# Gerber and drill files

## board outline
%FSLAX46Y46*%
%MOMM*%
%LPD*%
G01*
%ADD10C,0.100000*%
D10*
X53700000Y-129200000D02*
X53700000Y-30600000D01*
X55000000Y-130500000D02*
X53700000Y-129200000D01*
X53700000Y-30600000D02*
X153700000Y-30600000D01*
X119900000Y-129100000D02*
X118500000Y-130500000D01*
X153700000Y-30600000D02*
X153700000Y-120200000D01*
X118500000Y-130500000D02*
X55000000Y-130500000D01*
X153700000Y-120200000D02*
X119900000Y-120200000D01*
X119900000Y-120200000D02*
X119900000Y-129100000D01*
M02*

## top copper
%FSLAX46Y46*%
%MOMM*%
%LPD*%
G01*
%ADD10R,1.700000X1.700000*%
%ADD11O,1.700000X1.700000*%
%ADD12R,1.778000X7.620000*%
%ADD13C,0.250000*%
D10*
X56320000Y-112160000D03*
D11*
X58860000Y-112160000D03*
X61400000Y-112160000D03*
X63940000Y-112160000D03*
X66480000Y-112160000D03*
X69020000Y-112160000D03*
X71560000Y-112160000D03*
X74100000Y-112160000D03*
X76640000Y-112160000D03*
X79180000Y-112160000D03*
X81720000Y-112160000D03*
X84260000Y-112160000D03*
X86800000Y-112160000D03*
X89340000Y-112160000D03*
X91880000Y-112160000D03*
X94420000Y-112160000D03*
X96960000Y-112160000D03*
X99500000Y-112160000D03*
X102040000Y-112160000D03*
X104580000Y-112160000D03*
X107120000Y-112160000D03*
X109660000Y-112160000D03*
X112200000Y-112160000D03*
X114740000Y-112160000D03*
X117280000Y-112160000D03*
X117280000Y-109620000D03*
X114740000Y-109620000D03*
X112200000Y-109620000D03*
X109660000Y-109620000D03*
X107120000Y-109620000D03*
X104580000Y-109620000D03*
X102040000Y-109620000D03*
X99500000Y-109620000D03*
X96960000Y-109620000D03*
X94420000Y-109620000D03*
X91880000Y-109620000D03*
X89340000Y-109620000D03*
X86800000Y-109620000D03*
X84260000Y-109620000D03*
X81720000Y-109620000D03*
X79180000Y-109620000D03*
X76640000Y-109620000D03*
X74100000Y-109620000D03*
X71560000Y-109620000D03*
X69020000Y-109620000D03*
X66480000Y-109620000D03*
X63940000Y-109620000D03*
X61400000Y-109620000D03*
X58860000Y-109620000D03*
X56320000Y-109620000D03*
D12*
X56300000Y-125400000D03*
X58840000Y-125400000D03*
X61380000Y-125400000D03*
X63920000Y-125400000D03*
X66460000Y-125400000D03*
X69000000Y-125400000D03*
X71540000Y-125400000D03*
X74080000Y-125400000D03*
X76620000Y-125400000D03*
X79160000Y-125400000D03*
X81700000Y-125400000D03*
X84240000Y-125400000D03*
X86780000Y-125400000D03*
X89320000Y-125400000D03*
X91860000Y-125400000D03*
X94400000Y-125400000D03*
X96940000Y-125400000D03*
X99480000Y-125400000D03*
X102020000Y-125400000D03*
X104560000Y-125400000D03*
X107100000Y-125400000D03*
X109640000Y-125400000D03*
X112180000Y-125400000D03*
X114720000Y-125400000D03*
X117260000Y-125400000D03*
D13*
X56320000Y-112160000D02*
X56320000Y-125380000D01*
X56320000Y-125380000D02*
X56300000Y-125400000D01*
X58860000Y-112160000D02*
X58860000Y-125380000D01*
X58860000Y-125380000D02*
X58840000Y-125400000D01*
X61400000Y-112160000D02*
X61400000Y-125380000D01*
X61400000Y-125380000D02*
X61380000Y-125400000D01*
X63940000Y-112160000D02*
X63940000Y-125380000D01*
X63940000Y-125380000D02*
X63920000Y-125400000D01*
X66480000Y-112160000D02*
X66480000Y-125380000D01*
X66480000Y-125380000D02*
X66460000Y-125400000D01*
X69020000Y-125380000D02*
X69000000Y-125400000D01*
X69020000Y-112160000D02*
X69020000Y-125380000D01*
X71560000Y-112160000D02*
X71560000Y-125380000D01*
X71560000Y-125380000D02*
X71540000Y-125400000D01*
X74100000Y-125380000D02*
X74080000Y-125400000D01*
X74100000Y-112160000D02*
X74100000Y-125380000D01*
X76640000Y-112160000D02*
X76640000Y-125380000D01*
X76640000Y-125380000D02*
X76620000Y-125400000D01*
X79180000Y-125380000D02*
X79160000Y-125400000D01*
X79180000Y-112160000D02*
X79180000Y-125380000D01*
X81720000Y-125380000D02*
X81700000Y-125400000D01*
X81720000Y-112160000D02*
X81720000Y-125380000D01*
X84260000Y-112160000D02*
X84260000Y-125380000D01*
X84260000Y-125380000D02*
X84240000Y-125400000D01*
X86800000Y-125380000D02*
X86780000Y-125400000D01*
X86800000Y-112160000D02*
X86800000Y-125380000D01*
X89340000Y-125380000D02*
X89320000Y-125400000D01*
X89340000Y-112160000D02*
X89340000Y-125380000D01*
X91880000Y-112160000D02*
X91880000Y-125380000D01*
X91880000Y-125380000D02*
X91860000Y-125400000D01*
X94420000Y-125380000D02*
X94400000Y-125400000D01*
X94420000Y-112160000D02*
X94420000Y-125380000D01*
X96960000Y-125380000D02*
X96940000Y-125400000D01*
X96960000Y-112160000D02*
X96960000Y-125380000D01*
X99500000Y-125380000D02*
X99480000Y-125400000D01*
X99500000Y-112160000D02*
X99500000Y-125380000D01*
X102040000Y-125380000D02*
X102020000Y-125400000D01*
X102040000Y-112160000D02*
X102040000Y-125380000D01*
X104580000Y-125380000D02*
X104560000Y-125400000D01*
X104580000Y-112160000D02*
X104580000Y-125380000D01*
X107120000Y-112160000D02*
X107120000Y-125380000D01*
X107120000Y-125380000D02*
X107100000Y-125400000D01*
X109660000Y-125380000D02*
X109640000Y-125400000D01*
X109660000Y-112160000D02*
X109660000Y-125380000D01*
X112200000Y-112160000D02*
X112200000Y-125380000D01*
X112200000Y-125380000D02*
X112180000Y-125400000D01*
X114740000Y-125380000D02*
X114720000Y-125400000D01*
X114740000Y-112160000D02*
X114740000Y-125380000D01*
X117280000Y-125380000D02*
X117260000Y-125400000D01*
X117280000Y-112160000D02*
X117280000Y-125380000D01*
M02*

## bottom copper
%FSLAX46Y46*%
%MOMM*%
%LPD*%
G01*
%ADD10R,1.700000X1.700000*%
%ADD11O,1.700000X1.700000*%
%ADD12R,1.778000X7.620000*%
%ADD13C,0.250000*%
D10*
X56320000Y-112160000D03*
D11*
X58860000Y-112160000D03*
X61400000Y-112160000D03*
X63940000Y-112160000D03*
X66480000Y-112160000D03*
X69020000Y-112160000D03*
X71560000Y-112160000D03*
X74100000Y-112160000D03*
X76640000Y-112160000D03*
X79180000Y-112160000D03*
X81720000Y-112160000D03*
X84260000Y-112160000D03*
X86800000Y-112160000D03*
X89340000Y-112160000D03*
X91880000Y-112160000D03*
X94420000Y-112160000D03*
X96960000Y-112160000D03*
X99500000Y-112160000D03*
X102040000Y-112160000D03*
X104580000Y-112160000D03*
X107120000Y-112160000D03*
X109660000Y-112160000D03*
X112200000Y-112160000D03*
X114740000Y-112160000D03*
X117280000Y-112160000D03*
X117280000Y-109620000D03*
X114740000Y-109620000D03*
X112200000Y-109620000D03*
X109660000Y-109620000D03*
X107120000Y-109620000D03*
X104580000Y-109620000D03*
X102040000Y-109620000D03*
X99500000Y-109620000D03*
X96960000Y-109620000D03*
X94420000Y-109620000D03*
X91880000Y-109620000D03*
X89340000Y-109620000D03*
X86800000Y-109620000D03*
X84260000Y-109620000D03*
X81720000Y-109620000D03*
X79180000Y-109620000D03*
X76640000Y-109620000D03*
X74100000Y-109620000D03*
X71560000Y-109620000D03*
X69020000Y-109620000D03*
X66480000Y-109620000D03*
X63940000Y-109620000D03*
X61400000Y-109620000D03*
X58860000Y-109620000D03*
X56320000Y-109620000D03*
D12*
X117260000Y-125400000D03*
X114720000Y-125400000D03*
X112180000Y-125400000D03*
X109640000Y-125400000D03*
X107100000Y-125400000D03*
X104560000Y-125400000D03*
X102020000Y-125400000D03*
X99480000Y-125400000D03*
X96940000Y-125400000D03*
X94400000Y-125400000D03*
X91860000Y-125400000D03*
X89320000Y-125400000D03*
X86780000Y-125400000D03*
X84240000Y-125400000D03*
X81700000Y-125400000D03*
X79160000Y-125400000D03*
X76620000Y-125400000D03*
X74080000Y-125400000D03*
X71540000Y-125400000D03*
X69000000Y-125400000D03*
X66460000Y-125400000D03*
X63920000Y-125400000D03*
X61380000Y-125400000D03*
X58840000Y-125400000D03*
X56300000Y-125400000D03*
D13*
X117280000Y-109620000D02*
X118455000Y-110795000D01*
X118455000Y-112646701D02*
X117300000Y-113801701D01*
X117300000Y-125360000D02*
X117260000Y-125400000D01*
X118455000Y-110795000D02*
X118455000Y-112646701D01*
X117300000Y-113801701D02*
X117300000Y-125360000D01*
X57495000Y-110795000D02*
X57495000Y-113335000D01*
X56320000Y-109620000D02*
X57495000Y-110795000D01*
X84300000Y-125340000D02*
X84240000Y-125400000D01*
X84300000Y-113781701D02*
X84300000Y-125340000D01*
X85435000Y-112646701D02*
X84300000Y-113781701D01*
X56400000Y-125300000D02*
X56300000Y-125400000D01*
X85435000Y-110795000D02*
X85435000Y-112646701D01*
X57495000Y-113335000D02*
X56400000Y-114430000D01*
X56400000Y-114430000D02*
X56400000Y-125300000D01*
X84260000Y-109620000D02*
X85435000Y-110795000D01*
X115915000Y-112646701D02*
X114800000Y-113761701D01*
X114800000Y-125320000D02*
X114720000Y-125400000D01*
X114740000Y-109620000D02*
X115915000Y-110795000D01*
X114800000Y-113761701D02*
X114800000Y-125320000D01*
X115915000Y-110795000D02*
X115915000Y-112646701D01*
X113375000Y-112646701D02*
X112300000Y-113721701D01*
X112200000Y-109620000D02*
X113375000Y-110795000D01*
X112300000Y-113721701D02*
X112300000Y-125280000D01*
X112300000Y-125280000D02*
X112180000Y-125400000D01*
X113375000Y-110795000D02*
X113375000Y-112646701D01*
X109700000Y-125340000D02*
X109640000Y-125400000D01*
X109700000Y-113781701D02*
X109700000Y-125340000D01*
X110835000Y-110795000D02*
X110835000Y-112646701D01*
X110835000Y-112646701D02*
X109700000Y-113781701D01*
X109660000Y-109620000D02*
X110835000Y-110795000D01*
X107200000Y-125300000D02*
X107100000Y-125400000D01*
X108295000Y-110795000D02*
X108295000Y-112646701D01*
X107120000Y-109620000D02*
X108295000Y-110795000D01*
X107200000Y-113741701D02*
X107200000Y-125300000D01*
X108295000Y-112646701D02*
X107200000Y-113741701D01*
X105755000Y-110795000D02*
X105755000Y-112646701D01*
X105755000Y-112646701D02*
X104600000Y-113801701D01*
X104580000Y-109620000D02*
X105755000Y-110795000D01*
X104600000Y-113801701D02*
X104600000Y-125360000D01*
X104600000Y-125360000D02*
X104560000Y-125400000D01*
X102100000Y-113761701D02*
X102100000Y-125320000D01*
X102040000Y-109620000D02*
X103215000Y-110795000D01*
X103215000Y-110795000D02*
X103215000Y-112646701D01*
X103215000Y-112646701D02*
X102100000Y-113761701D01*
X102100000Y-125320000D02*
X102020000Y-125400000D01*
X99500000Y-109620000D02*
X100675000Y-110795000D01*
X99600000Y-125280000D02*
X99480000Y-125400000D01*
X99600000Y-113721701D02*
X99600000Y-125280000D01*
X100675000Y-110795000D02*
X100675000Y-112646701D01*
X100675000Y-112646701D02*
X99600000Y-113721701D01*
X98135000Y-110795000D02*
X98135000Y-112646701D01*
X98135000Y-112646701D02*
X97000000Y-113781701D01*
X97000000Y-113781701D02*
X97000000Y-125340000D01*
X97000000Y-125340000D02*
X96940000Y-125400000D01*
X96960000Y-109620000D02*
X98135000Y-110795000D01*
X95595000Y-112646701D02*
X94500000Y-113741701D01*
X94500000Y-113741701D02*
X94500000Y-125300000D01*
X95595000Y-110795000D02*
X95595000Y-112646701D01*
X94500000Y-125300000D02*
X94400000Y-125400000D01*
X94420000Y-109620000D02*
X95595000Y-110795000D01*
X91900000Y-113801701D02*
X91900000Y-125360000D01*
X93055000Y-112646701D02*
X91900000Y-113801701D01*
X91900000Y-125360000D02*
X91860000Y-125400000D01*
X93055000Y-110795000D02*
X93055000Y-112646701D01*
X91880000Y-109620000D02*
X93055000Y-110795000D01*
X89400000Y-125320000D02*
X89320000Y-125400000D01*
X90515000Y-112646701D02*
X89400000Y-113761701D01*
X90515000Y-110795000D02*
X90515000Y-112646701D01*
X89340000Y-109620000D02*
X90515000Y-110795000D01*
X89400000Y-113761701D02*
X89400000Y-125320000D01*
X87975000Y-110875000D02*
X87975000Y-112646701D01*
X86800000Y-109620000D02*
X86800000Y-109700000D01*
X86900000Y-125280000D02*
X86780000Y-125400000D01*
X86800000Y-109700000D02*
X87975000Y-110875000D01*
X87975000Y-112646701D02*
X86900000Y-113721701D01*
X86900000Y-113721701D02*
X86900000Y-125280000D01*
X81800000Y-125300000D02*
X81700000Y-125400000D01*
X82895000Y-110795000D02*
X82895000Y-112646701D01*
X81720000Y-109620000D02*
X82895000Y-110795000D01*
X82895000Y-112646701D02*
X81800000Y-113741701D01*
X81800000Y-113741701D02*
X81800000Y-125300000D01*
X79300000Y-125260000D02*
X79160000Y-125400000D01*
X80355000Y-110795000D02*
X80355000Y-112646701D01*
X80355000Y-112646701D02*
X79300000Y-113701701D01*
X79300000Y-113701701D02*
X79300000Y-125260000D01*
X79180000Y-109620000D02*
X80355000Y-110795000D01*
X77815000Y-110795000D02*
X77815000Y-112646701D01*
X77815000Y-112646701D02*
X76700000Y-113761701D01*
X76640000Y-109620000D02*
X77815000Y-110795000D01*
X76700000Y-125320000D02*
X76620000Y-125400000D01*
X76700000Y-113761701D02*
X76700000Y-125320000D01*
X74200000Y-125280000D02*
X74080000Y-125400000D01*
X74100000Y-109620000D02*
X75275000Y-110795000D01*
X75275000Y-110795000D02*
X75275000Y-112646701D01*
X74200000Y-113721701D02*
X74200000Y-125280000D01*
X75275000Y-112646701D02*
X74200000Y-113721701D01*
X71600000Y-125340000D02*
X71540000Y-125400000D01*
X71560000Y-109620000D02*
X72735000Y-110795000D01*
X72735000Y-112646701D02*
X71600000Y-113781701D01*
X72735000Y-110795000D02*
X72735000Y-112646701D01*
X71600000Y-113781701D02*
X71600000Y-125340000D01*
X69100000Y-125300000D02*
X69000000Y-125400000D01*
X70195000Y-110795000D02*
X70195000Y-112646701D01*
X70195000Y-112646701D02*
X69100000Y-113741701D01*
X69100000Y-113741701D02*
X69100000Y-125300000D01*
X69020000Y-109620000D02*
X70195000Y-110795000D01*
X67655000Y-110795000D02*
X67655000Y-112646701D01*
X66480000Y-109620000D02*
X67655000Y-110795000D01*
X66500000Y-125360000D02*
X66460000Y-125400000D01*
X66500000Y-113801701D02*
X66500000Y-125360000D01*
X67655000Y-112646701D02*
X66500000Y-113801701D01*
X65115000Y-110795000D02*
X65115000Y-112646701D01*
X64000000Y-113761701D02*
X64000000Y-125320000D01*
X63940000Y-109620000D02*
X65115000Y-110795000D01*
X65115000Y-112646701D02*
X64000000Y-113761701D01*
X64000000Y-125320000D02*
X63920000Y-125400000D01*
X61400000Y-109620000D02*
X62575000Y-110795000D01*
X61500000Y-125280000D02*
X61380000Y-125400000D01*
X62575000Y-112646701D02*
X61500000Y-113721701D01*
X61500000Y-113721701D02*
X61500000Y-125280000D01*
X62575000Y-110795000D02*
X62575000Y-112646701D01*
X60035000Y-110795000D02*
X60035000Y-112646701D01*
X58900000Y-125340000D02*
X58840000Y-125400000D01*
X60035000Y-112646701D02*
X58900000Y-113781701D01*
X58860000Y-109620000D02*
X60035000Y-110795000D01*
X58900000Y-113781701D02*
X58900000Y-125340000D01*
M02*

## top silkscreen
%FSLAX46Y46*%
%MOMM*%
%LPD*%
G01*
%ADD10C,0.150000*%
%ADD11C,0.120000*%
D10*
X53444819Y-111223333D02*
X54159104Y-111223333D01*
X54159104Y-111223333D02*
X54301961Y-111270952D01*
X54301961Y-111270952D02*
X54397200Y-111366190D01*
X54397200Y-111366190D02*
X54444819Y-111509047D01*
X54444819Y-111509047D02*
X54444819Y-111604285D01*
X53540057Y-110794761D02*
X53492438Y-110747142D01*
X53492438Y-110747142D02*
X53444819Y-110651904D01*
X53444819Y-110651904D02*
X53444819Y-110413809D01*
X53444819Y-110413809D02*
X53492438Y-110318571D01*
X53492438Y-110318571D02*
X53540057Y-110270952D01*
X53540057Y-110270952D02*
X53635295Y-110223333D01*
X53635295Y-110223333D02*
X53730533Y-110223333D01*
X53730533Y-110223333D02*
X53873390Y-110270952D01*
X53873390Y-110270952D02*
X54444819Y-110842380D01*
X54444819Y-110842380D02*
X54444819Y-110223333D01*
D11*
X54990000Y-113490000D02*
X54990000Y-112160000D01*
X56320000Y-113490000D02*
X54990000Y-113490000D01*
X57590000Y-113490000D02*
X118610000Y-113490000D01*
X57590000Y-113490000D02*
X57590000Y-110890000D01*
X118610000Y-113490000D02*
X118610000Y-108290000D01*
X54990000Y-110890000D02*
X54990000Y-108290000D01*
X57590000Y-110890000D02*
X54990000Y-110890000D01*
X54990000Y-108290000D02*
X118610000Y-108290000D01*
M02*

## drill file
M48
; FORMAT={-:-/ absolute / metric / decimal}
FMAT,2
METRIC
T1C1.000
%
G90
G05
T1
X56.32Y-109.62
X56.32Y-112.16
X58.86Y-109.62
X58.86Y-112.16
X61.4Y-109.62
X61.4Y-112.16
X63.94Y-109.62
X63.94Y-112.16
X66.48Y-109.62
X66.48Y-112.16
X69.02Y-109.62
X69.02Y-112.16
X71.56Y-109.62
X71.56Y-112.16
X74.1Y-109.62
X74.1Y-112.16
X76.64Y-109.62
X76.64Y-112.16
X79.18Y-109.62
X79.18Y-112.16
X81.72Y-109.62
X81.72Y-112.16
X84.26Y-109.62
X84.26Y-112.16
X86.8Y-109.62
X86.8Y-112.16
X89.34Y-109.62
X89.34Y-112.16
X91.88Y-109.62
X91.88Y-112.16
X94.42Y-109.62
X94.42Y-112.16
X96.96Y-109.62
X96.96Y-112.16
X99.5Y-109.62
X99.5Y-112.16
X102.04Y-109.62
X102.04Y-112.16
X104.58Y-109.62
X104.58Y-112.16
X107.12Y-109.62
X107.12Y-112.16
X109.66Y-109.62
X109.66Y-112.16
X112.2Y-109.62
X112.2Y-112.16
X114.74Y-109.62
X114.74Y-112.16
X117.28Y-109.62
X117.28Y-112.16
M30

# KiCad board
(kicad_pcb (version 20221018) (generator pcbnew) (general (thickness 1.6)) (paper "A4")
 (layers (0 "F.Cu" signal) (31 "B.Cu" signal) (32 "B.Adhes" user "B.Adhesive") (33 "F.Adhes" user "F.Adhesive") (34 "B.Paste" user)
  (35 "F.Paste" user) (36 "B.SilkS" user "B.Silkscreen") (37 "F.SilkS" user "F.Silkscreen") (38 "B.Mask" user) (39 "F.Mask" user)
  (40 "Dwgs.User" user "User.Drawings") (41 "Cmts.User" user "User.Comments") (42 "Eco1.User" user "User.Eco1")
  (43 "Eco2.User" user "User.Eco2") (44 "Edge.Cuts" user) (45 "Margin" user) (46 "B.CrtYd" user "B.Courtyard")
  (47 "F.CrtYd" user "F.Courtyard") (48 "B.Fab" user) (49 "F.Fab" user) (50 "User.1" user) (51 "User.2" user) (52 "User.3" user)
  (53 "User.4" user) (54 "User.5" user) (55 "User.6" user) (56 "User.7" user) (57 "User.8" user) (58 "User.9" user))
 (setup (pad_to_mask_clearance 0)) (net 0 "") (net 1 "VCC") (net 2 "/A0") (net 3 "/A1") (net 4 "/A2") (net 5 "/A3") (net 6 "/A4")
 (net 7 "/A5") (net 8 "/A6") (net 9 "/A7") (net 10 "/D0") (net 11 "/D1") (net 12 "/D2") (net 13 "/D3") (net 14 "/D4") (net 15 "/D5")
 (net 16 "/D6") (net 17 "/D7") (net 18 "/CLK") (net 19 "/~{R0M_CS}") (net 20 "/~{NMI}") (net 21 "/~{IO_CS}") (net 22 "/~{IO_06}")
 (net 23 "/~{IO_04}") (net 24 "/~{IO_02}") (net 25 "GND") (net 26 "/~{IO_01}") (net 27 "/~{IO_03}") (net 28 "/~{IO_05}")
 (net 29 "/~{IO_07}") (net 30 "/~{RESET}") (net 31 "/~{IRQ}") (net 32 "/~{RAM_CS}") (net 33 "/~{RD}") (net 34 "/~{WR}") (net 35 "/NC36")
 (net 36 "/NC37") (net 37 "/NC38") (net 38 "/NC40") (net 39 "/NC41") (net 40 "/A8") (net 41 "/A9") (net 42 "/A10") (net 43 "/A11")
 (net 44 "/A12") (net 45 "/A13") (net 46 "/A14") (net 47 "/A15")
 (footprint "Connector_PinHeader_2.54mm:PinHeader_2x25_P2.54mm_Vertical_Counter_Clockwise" (layer "F.Cu") (at 56.32 112.16 90)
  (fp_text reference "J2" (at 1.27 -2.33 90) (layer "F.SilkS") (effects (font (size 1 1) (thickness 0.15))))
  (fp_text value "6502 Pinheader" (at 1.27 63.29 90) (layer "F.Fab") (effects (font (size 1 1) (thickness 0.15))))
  (fp_line (start -1.33 -1.33) (end 0 -1.33) (stroke (width 0.12) (type solid)) (layer "F.SilkS"))
  (fp_line (start -1.33 0) (end -1.33 -1.33) (stroke (width 0.12) (type solid)) (layer "F.SilkS"))
  (fp_line (start -1.33 1.27) (end -1.33 62.29) (stroke (width 0.12) (type solid)) (layer "F.SilkS"))
  (fp_line (start -1.33 1.27) (end 1.27 1.27) (stroke (width 0.12) (type solid)) (layer "F.SilkS"))
  (fp_line (start -1.33 62.29) (end 3.87 62.29) (stroke (width 0.12) (type solid)) (layer "F.SilkS"))
  (fp_line (start 1.27 -1.33) (end 3.87 -1.33) (stroke (width 0.12) (type solid)) (layer "F.SilkS"))
  (fp_line (start 1.27 1.27) (end 1.27 -1.33) (stroke (width 0.12) (type solid)) (layer "F.SilkS"))
  (fp_line (start 3.87 -1.33) (end 3.87 62.29) (stroke (width 0.12) (type solid)) (layer "F.SilkS"))
  (pad "1" thru_hole rect (at 0 0 90) (size 1.7 1.7) (drill 1) (layers "*.Cu" "*.Mask") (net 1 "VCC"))
  (pad "2" thru_hole oval (at 0 2.54 90) (size 1.7 1.7) (drill 1) (layers "*.Cu" "*.Mask") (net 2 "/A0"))
  (pad "3" thru_hole oval (at 0 5.08 90) (size 1.7 1.7) (drill 1) (layers "*.Cu" "*.Mask") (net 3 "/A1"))
  (pad "4" thru_hole oval (at 0 7.62 90) (size 1.7 1.7) (drill 1) (layers "*.Cu" "*.Mask") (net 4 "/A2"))
  (pad "5" thru_hole oval (at 0 10.16 90) (size 1.7 1.7) (drill 1) (layers "*.Cu" "*.Mask") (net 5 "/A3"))
  (pad "6" thru_hole oval (at 0 12.7 90) (size 1.7 1.7) (drill 1) (layers "*.Cu" "*.Mask") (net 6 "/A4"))
  (pad "7" thru_hole oval (at 0 15.24 90) (size 1.7 1.7) (drill 1) (layers "*.Cu" "*.Mask") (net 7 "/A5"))
  (pad "8" thru_hole oval (at 0 17.78 90) (size 1.7 1.7) (drill 1) (layers "*.Cu" "*.Mask") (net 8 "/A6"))
  (pad "9" thru_hole oval (at 0 20.32 90) (size 1.7 1.7) (drill 1) (layers "*.Cu" "*.Mask") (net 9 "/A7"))
  (pad "10" thru_hole oval (at 0 22.86 90) (size 1.7 1.7) (drill 1) (layers "*.Cu" "*.Mask") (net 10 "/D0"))
  (pad "11" thru_hole oval (at 0 25.4 90) (size 1.7 1.7) (drill 1) (layers "*.Cu" "*.Mask") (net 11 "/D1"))
  (pad "12" thru_hole oval (at 0 27.94 90) (size 1.7 1.7) (drill 1) (layers "*.Cu" "*.Mask") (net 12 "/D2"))
  (pad "13" thru_hole oval (at 0 30.48 90) (size 1.7 1.7) (drill 1) (layers "*.Cu" "*.Mask") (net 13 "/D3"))
  (pad "14" thru_hole oval (at 0 33.02 90) (size 1.7 1.7) (drill 1) (layers "*.Cu" "*.Mask") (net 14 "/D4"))
  (pad "15" thru_hole oval (at 0 35.56 90) (size 1.7 1.7) (drill 1) (layers "*.Cu" "*.Mask") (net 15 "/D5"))
  (pad "16" thru_hole oval (at 0 38.1 90) (size 1.7 1.7) (drill 1) (layers "*.Cu" "*.Mask") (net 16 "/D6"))
  (pad "17" thru_hole oval (at 0 40.64 90) (size 1.7 1.7) (drill 1) (layers "*.Cu" "*.Mask") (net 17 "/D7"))
  (pad "18" thru_hole oval (at 0 43.18 90) (size 1.7 1.7) (drill 1) (layers "*.Cu" "*.Mask") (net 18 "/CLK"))
  (pad "19" thru_hole oval (at 0 45.72 90) (size 1.7 1.7) (drill 1) (layers "*.Cu" "*.Mask") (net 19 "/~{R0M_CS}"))
  (pad "20" thru_hole oval (at 0 48.26 90) (size 1.7 1.7) (drill 1) (layers "*.Cu" "*.Mask") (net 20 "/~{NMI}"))
  (pad "21" thru_hole oval (at 0 50.8 90) (size 1.7 1.7) (drill 1) (layers "*.Cu" "*.Mask") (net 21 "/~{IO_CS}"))
  (pad "22" thru_hole oval (at 0 53.34 90) (size 1.7 1.7) (drill 1) (layers "*.Cu" "*.Mask") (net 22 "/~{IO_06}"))
  (pad "23" thru_hole oval (at 0 55.88 90) (size 1.7 1.7) (drill 1) (layers "*.Cu" "*.Mask") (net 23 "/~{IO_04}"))
  (pad "24" thru_hole oval (at 0 58.42 90) (size 1.7 1.7) (drill 1) (layers "*.Cu" "*.Mask") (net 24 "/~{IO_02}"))
  (pad "25" thru_hole oval (at 0 60.96 90) (size 1.7 1.7) (drill 1) (layers "*.Cu" "*.Mask") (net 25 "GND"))
  (pad "26" thru_hole oval (at 2.54 60.96 90) (size 1.7 1.7) (drill 1) (layers "*.Cu" "*.Mask") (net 1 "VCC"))
  (pad "27" thru_hole oval (at 2.54 58.42 90) (size 1.7 1.7) (drill 1) (layers "*.Cu" "*.Mask") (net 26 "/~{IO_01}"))
  (pad "28" thru_hole oval (at 2.54 55.88 90) (size 1.7 1.7) (drill 1) (layers "*.Cu" "*.Mask") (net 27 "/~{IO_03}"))
  (pad "29" thru_hole oval (at 2.54 53.34 90) (size 1.7 1.7) (drill 1) (layers "*.Cu" "*.Mask") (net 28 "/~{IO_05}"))
  (pad "30" thru_hole oval (at 2.54 50.8 90) (size 1.7 1.7) (drill 1) (layers "*.Cu" "*.Mask") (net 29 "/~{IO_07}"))
  (pad "31" thru_hole oval (at 2.54 48.26 90) (size 1.7 1.7) (drill 1) (layers "*.Cu" "*.Mask") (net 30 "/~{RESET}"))
  (pad "32" thru_hole oval (at 2.54 45.72 90) (size 1.7 1.7) (drill 1) (layers "*.Cu" "*.Mask") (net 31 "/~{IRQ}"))
  (pad "33" thru_hole oval (at 2.54 43.18 90) (size 1.7 1.7) (drill 1) (layers "*.Cu" "*.Mask") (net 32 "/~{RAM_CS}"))
  (pad "34" thru_hole oval (at 2.54 40.64 90) (size 1.7 1.7) (drill 1) (layers "*.Cu" "*.Mask") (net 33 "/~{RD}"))
  (pad "35" thru_hole oval (at 2.54 38.1 90) (size 1.7 1.7) (drill 1) (layers "*.Cu" "*.Mask") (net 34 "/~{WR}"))
  (pad "36" thru_hole oval (at 2.54 35.56 90) (size 1.7 1.7) (drill 1) (layers "*.Cu" "*.Mask") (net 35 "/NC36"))
  (pad "37" thru_hole oval (at 2.54 33.02 90) (size 1.7 1.7) (drill 1) (layers "*.Cu" "*.Mask") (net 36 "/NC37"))
  (pad "38" thru_hole oval (at 2.54 30.48 90) (size 1.7 1.7) (drill 1) (layers "*.Cu" "*.Mask") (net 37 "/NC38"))
  (pad "39" thru_hole oval (at 2.54 27.94 90) (size 1.7 1.7) (drill 1) (layers "*.Cu" "*.Mask") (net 25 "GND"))
  (pad "40" thru_hole oval (at 2.54 25.4 90) (size 1.7 1.7) (drill 1) (layers "*.Cu" "*.Mask") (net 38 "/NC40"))
  (pad "41" thru_hole oval (at 2.54 22.86 90) (size 1.7 1.7) (drill 1) (layers "*.Cu" "*.Mask") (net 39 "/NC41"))
  (pad "42" thru_hole oval (at 2.54 20.32 90) (size 1.7 1.7) (drill 1) (layers "*.Cu" "*.Mask") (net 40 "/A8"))
  (pad "43" thru_hole oval (at 2.54 17.78 90) (size 1.7 1.7) (drill 1) (layers "*.Cu" "*.Mask") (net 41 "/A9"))
  (pad "44" thru_hole oval (at 2.54 15.24 90) (size 1.7 1.7) (drill 1) (layers "*.Cu" "*.Mask") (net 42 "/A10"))
  (pad "45" thru_hole oval (at 2.54 12.7 90) (size 1.7 1.7) (drill 1) (layers "*.Cu" "*.Mask") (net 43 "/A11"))
  (pad "46" thru_hole oval (at 2.54 10.16 90) (size 1.7 1.7) (drill 1) (layers "*.Cu" "*.Mask") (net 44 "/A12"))
  (pad "47" thru_hole oval (at 2.54 7.62 90) (size 1.7 1.7) (drill 1) (layers "*.Cu" "*.Mask") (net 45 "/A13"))
  (pad "48" thru_hole oval (at 2.54 5.08 90) (size 1.7 1.7) (drill 1) (layers "*.Cu" "*.Mask") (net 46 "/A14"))
  (pad "49" thru_hole oval (at 2.54 2.54 90) (size 1.7 1.7) (drill 1) (layers "*.Cu" "*.Mask") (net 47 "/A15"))
  (pad "50" thru_hole oval (at 2.54 0 90) (size 1.7 1.7) (drill 1) (layers "*.Cu" "*.Mask") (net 25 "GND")))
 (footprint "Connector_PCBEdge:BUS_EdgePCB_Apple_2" (layer "F.Cu") (at 79.16 125.4)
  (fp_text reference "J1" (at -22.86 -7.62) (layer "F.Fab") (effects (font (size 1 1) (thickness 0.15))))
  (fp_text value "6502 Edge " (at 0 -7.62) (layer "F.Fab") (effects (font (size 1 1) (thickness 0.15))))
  (pad "1" connect rect (at -22.86 0 180) (size 1.778 7.62) (layers "F.Cu" "F.Mask") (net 1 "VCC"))
  (pad "2" connect rect (at -20.32 0 180) (size 1.778 7.62) (layers "F.Cu" "F.Mask") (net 2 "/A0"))
  (pad "3" connect rect (at -17.78 0 180) (size 1.778 7.62) (layers "F.Cu" "F.Mask") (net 3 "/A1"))
  (pad "4" connect rect (at -15.24 0 180) (size 1.778 7.62) (layers "F.Cu" "F.Mask") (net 4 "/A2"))
  (pad "5" connect rect (at -12.7 0 180) (size 1.778 7.62) (layers "F.Cu" "F.Mask") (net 5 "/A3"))
  (pad "6" connect rect (at -10.16 0 180) (size 1.778 7.62) (layers "F.Cu" "F.Mask") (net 6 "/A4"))
  (pad "7" connect rect (at -7.62 0 180) (size 1.778 7.62) (layers "F.Cu" "F.Mask") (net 7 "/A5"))
  (pad "8" connect rect (at -5.08 0 180) (size 1.778 7.62) (layers "F.Cu" "F.Mask") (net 8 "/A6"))
  (pad "9" connect rect (at -2.54 0 180) (size 1.778 7.62) (layers "F.Cu" "F.Mask") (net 9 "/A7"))
  (pad "10" connect rect (at 0 0 180) (size 1.778 7.62) (layers "F.Cu" "F.Mask") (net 10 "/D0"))
  (pad "11" connect rect (at 2.54 0 180) (size 1.778 7.62) (layers "F.Cu" "F.Mask") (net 11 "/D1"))
  (pad "12" connect rect (at 5.08 0 180) (size 1.778 7.62) (layers "F.Cu" "F.Mask") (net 12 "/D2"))
  (pad "13" connect rect (at 7.62 0 180) (size 1.778 7.62) (layers "F.Cu" "F.Mask") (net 13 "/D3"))
  (pad "14" connect rect (at 10.16 0 180) (size 1.778 7.62) (layers "F.Cu" "F.Mask") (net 14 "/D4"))
  (pad "15" connect rect (at 12.7 0 180) (size 1.778 7.62) (layers "F.Cu" "F.Mask") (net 15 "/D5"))
  (pad "16" connect rect (at 15.24 0 180) (size 1.778 7.62) (layers "F.Cu" "F.Mask") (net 16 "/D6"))
  (pad "17" connect rect (at 17.78 0 180) (size 1.778 7.62) (layers "F.Cu" "F.Mask") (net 17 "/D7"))
  (pad "18" connect rect (at 20.32 0 180) (size 1.778 7.62) (layers "F.Cu" "F.Mask") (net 18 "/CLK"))
  (pad "19" connect rect (at 22.86 0 180) (size 1.778 7.62) (layers "F.Cu" "F.Mask") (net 19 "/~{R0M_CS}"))
  (pad "20" connect rect (at 25.4 0 180) (size 1.778 7.62) (layers "F.Cu" "F.Mask") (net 20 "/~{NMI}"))
  (pad "21" connect rect (at 27.94 0 180) (size 1.778 7.62) (layers "F.Cu" "F.Mask") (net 21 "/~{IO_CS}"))
  (pad "22" connect rect (at 30.48 0 180) (size 1.778 7.62) (layers "F.Cu" "F.Mask") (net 22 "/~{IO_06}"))
  (pad "23" connect rect (at 33.02 0 180) (size 1.778 7.62) (layers "F.Cu" "F.Mask") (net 23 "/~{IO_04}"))
  (pad "24" connect rect (at 35.56 0 180) (size 1.778 7.62) (layers "F.Cu" "F.Mask") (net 24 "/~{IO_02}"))
  (pad "25" connect rect (at 38.1 0 180) (size 1.778 7.62) (layers "F.Cu" "F.Mask") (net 25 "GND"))
  (pad "26" connect rect (at 38.1 0 180) (size 1.778 7.62) (layers "B.Cu" "B.Mask") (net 1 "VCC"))
  (pad "27" connect rect (at 35.56 0 180) (size 1.778 7.62) (layers "B.Cu" "B.Mask") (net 26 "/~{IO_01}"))
  (pad "28" connect rect (at 33.02 0 180) (size 1.778 7.62) (layers "B.Cu" "B.Mask") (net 27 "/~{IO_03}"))
  (pad "29" connect rect (at 30.48 0 180) (size 1.778 7.62) (layers "B.Cu" "B.Mask") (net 28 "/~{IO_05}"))
  (pad "30" connect rect (at 27.94 0 180) (size 1.778 7.62) (layers "B.Cu" "B.Mask") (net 29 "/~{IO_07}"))
  (pad "31" connect rect (at 25.4 0 180) (size 1.778 7.62) (layers "B.Cu" "B.Mask") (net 30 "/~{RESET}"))
  (pad "32" connect rect (at 22.86 0 180) (size 1.778 7.62) (layers "B.Cu" "B.Mask") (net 31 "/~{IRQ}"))
  (pad "33" connect rect (at 20.32 0 180) (size 1.778 7.62) (layers "B.Cu" "B.Mask") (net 32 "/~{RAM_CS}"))
  (pad "34" connect rect (at 17.78 0 180) (size 1.778 7.62) (layers "B.Cu" "B.Mask") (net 33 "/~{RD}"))
  (pad "35" connect rect (at 15.24 0 180) (size 1.778 7.62) (layers "B.Cu" "B.Mask") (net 34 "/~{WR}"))
  (pad "36" connect rect (at 12.7 0 180) (size 1.778 7.62) (layers "B.Cu" "B.Mask") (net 35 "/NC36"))
  (pad "37" connect rect (at 10.16 0 180) (size 1.778 7.62) (layers "B.Cu" "B.Mask") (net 36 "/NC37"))
  (pad "38" connect rect (at 7.62 0 180) (size 1.778 7.62) (layers "B.Cu" "B.Mask") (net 37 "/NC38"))
  (pad "39" connect rect (at 5.08 0 180) (size 1.778 7.62) (layers "B.Cu" "B.Mask") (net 25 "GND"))
  (pad "40" connect rect (at 2.54 0 180) (size 1.778 7.62) (layers "B.Cu" "B.Mask") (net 38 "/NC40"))
  (pad "41" connect rect (at 0 0 180) (size 1.778 7.62) (layers "B.Cu" "B.Mask") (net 39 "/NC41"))
  (pad "42" connect rect (at -2.54 0 180) (size 1.778 7.62) (layers "B.Cu" "B.Mask") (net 40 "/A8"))
  (pad "43" connect rect (at -5.08 0 180) (size 1.778 7.62) (layers "B.Cu" "B.Mask") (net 41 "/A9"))
  (pad "44" connect rect (at -7.62 0 180) (size 1.778 7.62) (layers "B.Cu" "B.Mask") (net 42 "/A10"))
  (pad "45" connect rect (at -10.16 0 180) (size 1.778 7.62) (layers "B.Cu" "B.Mask") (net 43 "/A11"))
  (pad "46" connect rect (at -12.7 0 180) (size 1.778 7.62) (layers "B.Cu" "B.Mask") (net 44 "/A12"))
  (pad "47" connect rect (at -15.24 0 180) (size 1.778 7.62) (layers "B.Cu" "B.Mask") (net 45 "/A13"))
  (pad "48" connect rect (at -17.78 0 180) (size 1.778 7.62) (layers "B.Cu" "B.Mask") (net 46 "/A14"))
  (pad "49" connect rect (at -20.32 0 180) (size 1.778 7.62) (layers "B.Cu" "B.Mask") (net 47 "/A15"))
  (pad "50" connect rect (at -22.86 0 180) (size 1.778 7.62) (layers "B.Cu" "B.Mask") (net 25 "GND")))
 (gr_line (start 53.7 129.2) (end 53.7 30.6) (stroke (width 0.1) (type default)) (layer "Edge.Cuts"))
 (gr_line (start 55 130.5) (end 53.7 129.2) (stroke (width 0.1) (type default)) (layer "Edge.Cuts"))
 (gr_line (start 53.7 30.6) (end 153.7 30.6) (stroke (width 0.1) (type default)) (layer "Edge.Cuts"))
 (gr_line (start 119.9 129.1) (end 118.5 130.5) (stroke (width 0.1) (type default)) (layer "Edge.Cuts"))
 (gr_line (start 153.7 30.6) (end 153.7 120.2) (stroke (width 0.1) (type default)) (layer "Edge.Cuts"))
 (gr_line (start 118.5 130.5) (end 55 130.5) (stroke (width 0.1) (type default)) (layer "Edge.Cuts"))
 (gr_line (start 153.7 120.2) (end 119.9 120.2) (stroke (width 0.1) (type default)) (layer "Edge.Cuts"))
 (gr_line (start 119.9 120.2) (end 119.9 129.1) (stroke (width 0.1) (type default)) (layer "Edge.Cuts"))
 (segment (start 56.32 112.16) (end 56.32 125.38) (width 0.25) (layer "F.Cu") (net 1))
 (segment (start 56.32 125.38) (end 56.3 125.4) (width 0.25) (layer "F.Cu") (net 1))
 (segment (start 117.28 109.62) (end 118.455 110.795) (width 0.25) (layer "B.Cu") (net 1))
 (segment (start 118.455 112.646701) (end 117.3 113.801701) (width 0.25) (layer "B.Cu") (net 1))
 (segment (start 117.3 125.36) (end 117.26 125.4) (width 0.25) (layer "B.Cu") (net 1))
 (segment (start 118.455 110.795) (end 118.455 112.646701) (width 0.25) (layer "B.Cu") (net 1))
 (segment (start 117.3 113.801701) (end 117.3 125.36) (width 0.25) (layer "B.Cu") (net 1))
 (segment (start 58.86 112.16) (end 58.86 125.38) (width 0.25) (layer "F.Cu") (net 2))
 (segment (start 58.86 125.38) (end 58.84 125.4) (width 0.25) (layer "F.Cu") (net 2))
 (segment (start 61.4 112.16) (end 61.4 125.38) (width 0.25) (layer "F.Cu") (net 3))
 (segment (start 61.4 125.38) (end 61.38 125.4) (width 0.25) (layer "F.Cu") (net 3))
 (segment (start 63.94 112.16) (end 63.94 125.38) (width 0.25) (layer "F.Cu") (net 4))
 (segment (start 63.94 125.38) (end 63.92 125.4) (width 0.25) (layer "F.Cu") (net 4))
 (segment (start 66.48 112.16) (end 66.48 125.38) (width 0.25) (layer "F.Cu") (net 5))
 (segment (start 66.48 125.38) (end 66.46 125.4) (width 0.25) (layer "F.Cu") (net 5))
 (segment (start 69.02 125.38) (end 69 125.4) (width 0.25) (layer "F.Cu") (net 6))
 (segment (start 69.02 112.16) (end 69.02 125.38) (width 0.25) (layer "F.Cu") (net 6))
 (segment (start 71.56 112.16) (end 71.56 125.38) (width 0.25) (layer "F.Cu") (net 7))
 (segment (start 71.56 125.38) (end 71.54 125.4) (width 0.25) (layer "F.Cu") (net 7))
 (segment (start 74.1 125.38) (end 74.08 125.4) (width 0.25) (layer "F.Cu") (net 8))
 (segment (start 74.1 112.16) (end 74.1 125.38) (width 0.25) (layer "F.Cu") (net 8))
 (segment (start 76.64 112.16) (end 76.64 125.38) (width 0.25) (layer "F.Cu") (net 9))
 (segment (start 76.64 125.38) (end 76.62 125.4) (width 0.25) (layer "F.Cu") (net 9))
 (segment (start 79.18 125.38) (end 79.16 125.4) (width 0.25) (layer "F.Cu") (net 10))
 (segment (start 79.18 112.16) (end 79.18 125.38) (width 0.25) (layer "F.Cu") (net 10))
 (segment (start 81.72 125.38) (end 81.7 125.4) (width 0.25) (layer "F.Cu") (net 11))
 (segment (start 81.72 112.16) (end 81.72 125.38) (width 0.25) (layer "F.Cu") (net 11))
 (segment (start 84.26 112.16) (end 84.26 125.38) (width 0.25) (layer "F.Cu") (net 12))
 (segment (start 84.26 125.38) (end 84.24 125.4) (width 0.25) (layer "F.Cu") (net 12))
 (segment (start 86.8 125.38) (end 86.78 125.4) (width 0.25) (layer "F.Cu") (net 13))
 (segment (start 86.8 112.16) (end 86.8 125.38) (width 0.25) (layer "F.Cu") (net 13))
 (segment (start 89.34 125.38) (end 89.32 125.4) (width 0.25) (layer "F.Cu") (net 14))
 (segment (start 89.34 112.16) (end 89.34 125.38) (width 0.25) (layer "F.Cu") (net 14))
 (segment (start 91.88 112.16) (end 91.88 125.38) (width 0.25) (layer "F.Cu") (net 15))
 (segment (start 91.88 125.38) (end 91.86 125.4) (width 0.25) (layer "F.Cu") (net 15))
 (segment (start 94.42 125.38) (end 94.4 125.4) (width 0.25) (layer "F.Cu") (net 16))
 (segment (start 94.42 112.16) (end 94.42 125.38) (width 0.25) (layer "F.Cu") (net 16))
 (segment (start 96.96 125.38) (end 96.94 125.4) (width 0.25) (layer "F.Cu") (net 17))
 (segment (start 96.96 112.16) (end 96.96 125.38) (width 0.25) (layer "F.Cu") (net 17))
 (segment (start 99.5 125.38) (end 99.48 125.4) (width 0.25) (layer "F.Cu") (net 18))
 (segment (start 99.5 112.16) (end 99.5 125.38) (width 0.25) (layer "F.Cu") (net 18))
 (segment (start 102.04 125.38) (end 102.02 125.4) (width 0.25) (layer "F.Cu") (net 19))
 (segment (start 102.04 112.16) (end 102.04 125.38) (width 0.25) (layer "F.Cu") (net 19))
 (segment (start 104.58 125.38) (end 104.56 125.4) (width 0.25) (layer "F.Cu") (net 20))
 (segment (start 104.58 112.16) (end 104.58 125.38) (width 0.25) (layer "F.Cu") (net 20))
 (segment (start 107.12 112.16) (end 107.12 125.38) (width 0.25) (layer "F.Cu") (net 21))
 (segment (start 107.12 125.38) (end 107.1 125.4) (width 0.25) (layer "F.Cu") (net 21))
 (segment (start 109.66 125.38) (end 109.64 125.4) (width 0.25) (layer "F.Cu") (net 22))
 (segment (start 109.66 112.16) (end 109.66 125.38) (width 0.25) (layer "F.Cu") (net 22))
 (segment (start 112.2 112.16) (end 112.2 125.38) (width 0.25) (layer "F.Cu") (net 23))
 (segment (start 112.2 125.38) (end 112.18 125.4) (width 0.25) (layer "F.Cu") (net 23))
 (segment (start 114.74 125.38) (end 114.72 125.4) (width 0.25) (layer "F.Cu") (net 24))
 (segment (start 114.74 112.16) (end 114.74 125.38) (width 0.25) (layer "F.Cu") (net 24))
 (segment (start 117.28 125.38) (end 117.26 125.4) (width 0.25) (layer "F.Cu") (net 25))
 (segment (start 117.28 112.16) (end 117.28 125.38) (width 0.25) (layer "F.Cu") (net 25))
 (segment (start 57.495 110.795) (end 57.495 113.335) (width 0.25) (layer "B.Cu") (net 25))
 (segment (start 56.32 109.62) (end 57.495 110.795) (width 0.25) (layer "B.Cu") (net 25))
 (segment (start 84.3 125.34) (end 84.24 125.4) (width 0.25) (layer "B.Cu") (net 25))
 (segment (start 84.3 113.781701) (end 84.3 125.34) (width 0.25) (layer "B.Cu") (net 25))
 (segment (start 85.435 112.646701) (end 84.3 113.781701) (width 0.25) (layer "B.Cu") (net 25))
 (segment (start 56.4 125.3) (end 56.3 125.4) (width 0.25) (layer "B.Cu") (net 25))
 (segment (start 85.435 110.795) (end 85.435 112.646701) (width 0.25) (layer "B.Cu") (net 25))
 (segment (start 57.495 113.335) (end 56.4 114.43) (width 0.25) (layer "B.Cu") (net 25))
 (segment (start 56.4 114.43) (end 56.4 125.3) (width 0.25) (layer "B.Cu") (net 25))
 (segment (start 84.26 109.62) (end 85.435 110.795) (width 0.25) (layer "B.Cu") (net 25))
 (segment (start 115.915 112.646701) (end 114.8 113.761701) (width 0.25) (layer "B.Cu") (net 26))
 (segment (start 114.8 125.32) (end 114.72 125.4) (width 0.25) (layer "B.Cu") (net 26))
 (segment (start 114.74 109.62) (end 115.915 110.795) (width 0.25) (layer "B.Cu") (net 26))
 (segment (start 114.8 113.761701) (end 114.8 125.32) (width 0.25) (layer "B.Cu") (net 26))
 (segment (start 115.915 110.795) (end 115.915 112.646701) (width 0.25) (layer "B.Cu") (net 26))
 (segment (start 113.375 112.646701) (end 112.3 113.721701) (width 0.25) (layer "B.Cu") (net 27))
 (segment (start 112.2 109.62) (end 113.375 110.795) (width 0.25) (layer "B.Cu") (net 27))
 (segment (start 112.3 113.721701) (end 112.3 125.28) (width 0.25) (layer "B.Cu") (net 27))
 (segment (start 112.3 125.28) (end 112.18 125.4) (width 0.25) (layer "B.Cu") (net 27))
 (segment (start 113.375 110.795) (end 113.375 112.646701) (width 0.25) (layer "B.Cu") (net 27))
 (segment (start 109.7 125.34) (end 109.64 125.4) (width 0.25) (layer "B.Cu") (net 28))
 (segment (start 109.7 113.781701) (end 109.7 125.34) (width 0.25) (layer "B.Cu") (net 28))
 (segment (start 110.835 110.795) (end 110.835 112.646701) (width 0.25) (layer "B.Cu") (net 28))
 (segment (start 110.835 112.646701) (end 109.7 113.781701) (width 0.25) (layer "B.Cu") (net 28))
 (segment (start 109.66 109.62) (end 110.835 110.795) (width 0.25) (layer "B.Cu") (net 28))
 (segment (start 107.2 125.3) (end 107.1 125.4) (width 0.25) (layer "B.Cu") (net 29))
 (segment (start 108.295 110.795) (end 108.295 112.646701) (width 0.25) (layer "B.Cu") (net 29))
 (segment (start 107.12 109.62) (end 108.295 110.795) (width 0.25) (layer "B.Cu") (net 29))
 (segment (start 107.2 113.741701) (end 107.2 125.3) (width 0.25) (layer "B.Cu") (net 29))
 (segment (start 108.295 112.646701) (end 107.2 113.741701) (width 0.25) (layer "B.Cu") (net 29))
 (segment (start 105.755 110.795) (end 105.755 112.646701) (width 0.25) (layer "B.Cu") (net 30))
 (segment (start 105.755 112.646701) (end 104.6 113.801701) (width 0.25) (layer "B.Cu") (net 30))
 (segment (start 104.58 109.62) (end 105.755 110.795) (width 0.25) (layer "B.Cu") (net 30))
 (segment (start 104.6 113.801701) (end 104.6 125.36) (width 0.25) (layer "B.Cu") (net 30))
 (segment (start 104.6 125.36) (end 104.56 125.4) (width 0.25) (layer "B.Cu") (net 30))
 (segment (start 102.1 113.761701) (end 102.1 125.32) (width 0.25) (layer "B.Cu") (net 31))
 (segment (start 102.04 109.62) (end 103.215 110.795) (width 0.25) (layer "B.Cu") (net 31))
 (segment (start 103.215 110.795) (end 103.215 112.646701) (width 0.25) (layer "B.Cu") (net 31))
 (segment (start 103.215 112.646701) (end 102.1 113.761701) (width 0.25) (layer "B.Cu") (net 31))
 (segment (start 102.1 125.32) (end 102.02 125.4) (width 0.25) (layer "B.Cu") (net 31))
 (segment (start 99.5 109.62) (end 100.675 110.795) (width 0.25) (layer "B.Cu") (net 32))
 (segment (start 99.6 125.28) (end 99.48 125.4) (width 0.25) (layer "B.Cu") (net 32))
 (segment (start 99.6 113.721701) (end 99.6 125.28) (width 0.25) (layer "B.Cu") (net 32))
 (segment (start 100.675 110.795) (end 100.675 112.646701) (width 0.25) (layer "B.Cu") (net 32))
 (segment (start 100.675 112.646701) (end 99.6 113.721701) (width 0.25) (layer "B.Cu") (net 32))
 (segment (start 98.135 110.795) (end 98.135 112.646701) (width 0.25) (layer "B.Cu") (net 33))
 (segment (start 98.135 112.646701) (end 97 113.781701) (width 0.25) (layer "B.Cu") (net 33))
 (segment (start 97 113.781701) (end 97 125.34) (width 0.25) (layer "B.Cu") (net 33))
 (segment (start 97 125.34) (end 96.94 125.4) (width 0.25) (layer "B.Cu") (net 33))
 (segment (start 96.96 109.62) (end 98.135 110.795) (width 0.25) (layer "B.Cu") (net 33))
 (segment (start 95.595 112.646701) (end 94.5 113.741701) (width 0.25) (layer "B.Cu") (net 34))
 (segment (start 94.5 113.741701) (end 94.5 125.3) (width 0.25) (layer "B.Cu") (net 34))
 (segment (start 95.595 110.795) (end 95.595 112.646701) (width 0.25) (layer "B.Cu") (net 34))
 (segment (start 94.5 125.3) (end 94.4 125.4) (width 0.25) (layer "B.Cu") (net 34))
 (segment (start 94.42 109.62) (end 95.595 110.795) (width 0.25) (layer "B.Cu") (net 34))
 (segment (start 91.9 113.801701) (end 91.9 125.36) (width 0.25) (layer "B.Cu") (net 35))
 (segment (start 93.055 112.646701) (end 91.9 113.801701) (width 0.25) (layer "B.Cu") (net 35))
 (segment (start 91.9 125.36) (end 91.86 125.4) (width 0.25) (layer "B.Cu") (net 35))
 (segment (start 93.055 110.795) (end 93.055 112.646701) (width 0.25) (layer "B.Cu") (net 35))
 (segment (start 91.88 109.62) (end 93.055 110.795) (width 0.25) (layer "B.Cu") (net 35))
 (segment (start 89.4 125.32) (end 89.32 125.4) (width 0.25) (layer "B.Cu") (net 36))
 (segment (start 90.515 112.646701) (end 89.4 113.761701) (width 0.25) (layer "B.Cu") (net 36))
 (segment (start 90.515 110.795) (end 90.515 112.646701) (width 0.25) (layer "B.Cu") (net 36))
 (segment (start 89.34 109.62) (end 90.515 110.795) (width 0.25) (layer "B.Cu") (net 36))
 (segment (start 89.4 113.761701) (end 89.4 125.32) (width 0.25) (layer "B.Cu") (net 36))
 (segment (start 87.975 110.875) (end 87.975 112.646701) (width 0.25) (layer "B.Cu") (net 37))
 (segment (start 86.8 109.62) (end 86.8 109.7) (width 0.25) (layer "B.Cu") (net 37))
 (segment (start 86.9 125.28) (end 86.78 125.4) (width 0.25) (layer "B.Cu") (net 37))
 (segment (start 86.8 109.7) (end 87.975 110.875) (width 0.25) (layer "B.Cu") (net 37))
 (segment (start 87.975 112.646701) (end 86.9 113.721701) (width 0.25) (layer "B.Cu") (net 37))
 (segment (start 86.9 113.721701) (end 86.9 125.28) (width 0.25) (layer "B.Cu") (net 37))
 (segment (start 81.8 125.3) (end 81.7 125.4) (width 0.25) (layer "B.Cu") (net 38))
 (segment (start 82.895 110.795) (end 82.895 112.646701) (width 0.25) (layer "B.Cu") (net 38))
 (segment (start 81.72 109.62) (end 82.895 110.795) (width 0.25) (layer "B.Cu") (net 38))
 (segment (start 82.895 112.646701) (end 81.8 113.741701) (width 0.25) (layer "B.Cu") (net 38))
 (segment (start 81.8 113.741701) (end 81.8 125.3) (width 0.25) (layer "B.Cu") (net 38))
 (segment (start 79.3 125.26) (end 79.16 125.4) (width 0.25) (layer "B.Cu") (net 39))
 (segment (start 80.355 110.795) (end 80.355 112.646701) (width 0.25) (layer "B.Cu") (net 39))
 (segment (start 80.355 112.646701) (end 79.3 113.701701) (width 0.25) (layer "B.Cu") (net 39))
 (segment (start 79.3 113.701701) (end 79.3 125.26) (width 0.25) (layer "B.Cu") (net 39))
 (segment (start 79.18 109.62) (end 80.355 110.795) (width 0.25) (layer "B.Cu") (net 39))
 (segment (start 77.815 110.795) (end 77.815 112.646701) (width 0.25) (layer "B.Cu") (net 40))
 (segment (start 77.815 112.646701) (end 76.7 113.761701) (width 0.25) (layer "B.Cu") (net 40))
 (segment (start 76.64 109.62) (end 77.815 110.795) (width 0.25) (layer "B.Cu") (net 40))
 (segment (start 76.7 125.32) (end 76.62 125.4) (width 0.25) (layer "B.Cu") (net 40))
 (segment (start 76.7 113.761701) (end 76.7 125.32) (width 0.25) (layer "B.Cu") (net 40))
 (segment (start 74.2 125.28) (end 74.08 125.4) (width 0.25) (layer "B.Cu") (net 41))
 (segment (start 74.1 109.62) (end 75.275 110.795) (width 0.25) (layer "B.Cu") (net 41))
 (segment (start 75.275 110.795) (end 75.275 112.646701) (width 0.25) (layer "B.Cu") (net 41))
 (segment (start 74.2 113.721701) (end 74.2 125.28) (width 0.25) (layer "B.Cu") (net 41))
 (segment (start 75.275 112.646701) (end 74.2 113.721701) (width 0.25) (layer "B.Cu") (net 41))
 (segment (start 71.6 125.34) (end 71.54 125.4) (width 0.25) (layer "B.Cu") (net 42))
 (segment (start 71.56 109.62) (end 72.735 110.795) (width 0.25) (layer "B.Cu") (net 42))
 (segment (start 72.735 112.646701) (end 71.6 113.781701) (width 0.25) (layer "B.Cu") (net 42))
 (segment (start 72.735 110.795) (end 72.735 112.646701) (width 0.25) (layer "B.Cu") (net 42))
 (segment (start 71.6 113.781701) (end 71.6 125.34) (width 0.25) (layer "B.Cu") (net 42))
 (segment (start 69.1 125.3) (end 69 125.4) (width 0.25) (layer "B.Cu") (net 43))
 (segment (start 70.195 110.795) (end 70.195 112.646701) (width 0.25) (layer "B.Cu") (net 43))
 (segment (start 70.195 112.646701) (end 69.1 113.741701) (width 0.25) (layer "B.Cu") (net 43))
 (segment (start 69.1 113.741701) (end 69.1 125.3) (width 0.25) (layer "B.Cu") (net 43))
 (segment (start 69.02 109.62) (end 70.195 110.795) (width 0.25) (layer "B.Cu") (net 43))
 (segment (start 67.655 110.795) (end 67.655 112.646701) (width 0.25) (layer "B.Cu") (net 44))
 (segment (start 66.48 109.62) (end 67.655 110.795) (width 0.25) (layer "B.Cu") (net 44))
 (segment (start 66.5 125.36) (end 66.46 125.4) (width 0.25) (layer "B.Cu") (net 44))
 (segment (start 66.5 113.801701) (end 66.5 125.36) (width 0.25) (layer "B.Cu") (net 44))
 (segment (start 67.655 112.646701) (end 66.5 113.801701) (width 0.25) (layer "B.Cu") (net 44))
 (segment (start 65.115 110.795) (end 65.115 112.646701) (width 0.25) (layer "B.Cu") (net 45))
 (segment (start 64 113.761701) (end 64 125.32) (width 0.25) (layer "B.Cu") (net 45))
 (segment (start 63.94 109.62) (end 65.115 110.795) (width 0.25) (layer "B.Cu") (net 45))
 (segment (start 65.115 112.646701) (end 64 113.761701) (width 0.25) (layer "B.Cu") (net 45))
 (segment (start 64 125.32) (end 63.92 125.4) (width 0.25) (layer "B.Cu") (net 45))
 (segment (start 61.4 109.62) (end 62.575 110.795) (width 0.25) (layer "B.Cu") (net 46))
 (segment (start 61.5 125.28) (end 61.38 125.4) (width 0.25) (layer "B.Cu") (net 46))
 (segment (start 62.575 112.646701) (end 61.5 113.721701) (width 0.25) (layer "B.Cu") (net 46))
 (segment (start 61.5 113.721701) (end 61.5 125.28) (width 0.25) (layer "B.Cu") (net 46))
 (segment (start 62.575 110.795) (end 62.575 112.646701) (width 0.25) (layer "B.Cu") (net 46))
 (segment (start 60.035 110.795) (end 60.035 112.646701) (width 0.25) (layer "B.Cu") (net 47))
 (segment (start 58.9 125.34) (end 58.84 125.4) (width 0.25) (layer "B.Cu") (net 47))
 (segment (start 60.035 112.646701) (end 58.9 113.781701) (width 0.25) (layer "B.Cu") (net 47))
 (segment (start 58.86 109.62) (end 60.035 110.795) (width 0.25) (layer "B.Cu") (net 47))
 (segment (start 58.9 113.781701) (end 58.9 125.34) (width 0.25) (layer "B.Cu") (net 47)))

